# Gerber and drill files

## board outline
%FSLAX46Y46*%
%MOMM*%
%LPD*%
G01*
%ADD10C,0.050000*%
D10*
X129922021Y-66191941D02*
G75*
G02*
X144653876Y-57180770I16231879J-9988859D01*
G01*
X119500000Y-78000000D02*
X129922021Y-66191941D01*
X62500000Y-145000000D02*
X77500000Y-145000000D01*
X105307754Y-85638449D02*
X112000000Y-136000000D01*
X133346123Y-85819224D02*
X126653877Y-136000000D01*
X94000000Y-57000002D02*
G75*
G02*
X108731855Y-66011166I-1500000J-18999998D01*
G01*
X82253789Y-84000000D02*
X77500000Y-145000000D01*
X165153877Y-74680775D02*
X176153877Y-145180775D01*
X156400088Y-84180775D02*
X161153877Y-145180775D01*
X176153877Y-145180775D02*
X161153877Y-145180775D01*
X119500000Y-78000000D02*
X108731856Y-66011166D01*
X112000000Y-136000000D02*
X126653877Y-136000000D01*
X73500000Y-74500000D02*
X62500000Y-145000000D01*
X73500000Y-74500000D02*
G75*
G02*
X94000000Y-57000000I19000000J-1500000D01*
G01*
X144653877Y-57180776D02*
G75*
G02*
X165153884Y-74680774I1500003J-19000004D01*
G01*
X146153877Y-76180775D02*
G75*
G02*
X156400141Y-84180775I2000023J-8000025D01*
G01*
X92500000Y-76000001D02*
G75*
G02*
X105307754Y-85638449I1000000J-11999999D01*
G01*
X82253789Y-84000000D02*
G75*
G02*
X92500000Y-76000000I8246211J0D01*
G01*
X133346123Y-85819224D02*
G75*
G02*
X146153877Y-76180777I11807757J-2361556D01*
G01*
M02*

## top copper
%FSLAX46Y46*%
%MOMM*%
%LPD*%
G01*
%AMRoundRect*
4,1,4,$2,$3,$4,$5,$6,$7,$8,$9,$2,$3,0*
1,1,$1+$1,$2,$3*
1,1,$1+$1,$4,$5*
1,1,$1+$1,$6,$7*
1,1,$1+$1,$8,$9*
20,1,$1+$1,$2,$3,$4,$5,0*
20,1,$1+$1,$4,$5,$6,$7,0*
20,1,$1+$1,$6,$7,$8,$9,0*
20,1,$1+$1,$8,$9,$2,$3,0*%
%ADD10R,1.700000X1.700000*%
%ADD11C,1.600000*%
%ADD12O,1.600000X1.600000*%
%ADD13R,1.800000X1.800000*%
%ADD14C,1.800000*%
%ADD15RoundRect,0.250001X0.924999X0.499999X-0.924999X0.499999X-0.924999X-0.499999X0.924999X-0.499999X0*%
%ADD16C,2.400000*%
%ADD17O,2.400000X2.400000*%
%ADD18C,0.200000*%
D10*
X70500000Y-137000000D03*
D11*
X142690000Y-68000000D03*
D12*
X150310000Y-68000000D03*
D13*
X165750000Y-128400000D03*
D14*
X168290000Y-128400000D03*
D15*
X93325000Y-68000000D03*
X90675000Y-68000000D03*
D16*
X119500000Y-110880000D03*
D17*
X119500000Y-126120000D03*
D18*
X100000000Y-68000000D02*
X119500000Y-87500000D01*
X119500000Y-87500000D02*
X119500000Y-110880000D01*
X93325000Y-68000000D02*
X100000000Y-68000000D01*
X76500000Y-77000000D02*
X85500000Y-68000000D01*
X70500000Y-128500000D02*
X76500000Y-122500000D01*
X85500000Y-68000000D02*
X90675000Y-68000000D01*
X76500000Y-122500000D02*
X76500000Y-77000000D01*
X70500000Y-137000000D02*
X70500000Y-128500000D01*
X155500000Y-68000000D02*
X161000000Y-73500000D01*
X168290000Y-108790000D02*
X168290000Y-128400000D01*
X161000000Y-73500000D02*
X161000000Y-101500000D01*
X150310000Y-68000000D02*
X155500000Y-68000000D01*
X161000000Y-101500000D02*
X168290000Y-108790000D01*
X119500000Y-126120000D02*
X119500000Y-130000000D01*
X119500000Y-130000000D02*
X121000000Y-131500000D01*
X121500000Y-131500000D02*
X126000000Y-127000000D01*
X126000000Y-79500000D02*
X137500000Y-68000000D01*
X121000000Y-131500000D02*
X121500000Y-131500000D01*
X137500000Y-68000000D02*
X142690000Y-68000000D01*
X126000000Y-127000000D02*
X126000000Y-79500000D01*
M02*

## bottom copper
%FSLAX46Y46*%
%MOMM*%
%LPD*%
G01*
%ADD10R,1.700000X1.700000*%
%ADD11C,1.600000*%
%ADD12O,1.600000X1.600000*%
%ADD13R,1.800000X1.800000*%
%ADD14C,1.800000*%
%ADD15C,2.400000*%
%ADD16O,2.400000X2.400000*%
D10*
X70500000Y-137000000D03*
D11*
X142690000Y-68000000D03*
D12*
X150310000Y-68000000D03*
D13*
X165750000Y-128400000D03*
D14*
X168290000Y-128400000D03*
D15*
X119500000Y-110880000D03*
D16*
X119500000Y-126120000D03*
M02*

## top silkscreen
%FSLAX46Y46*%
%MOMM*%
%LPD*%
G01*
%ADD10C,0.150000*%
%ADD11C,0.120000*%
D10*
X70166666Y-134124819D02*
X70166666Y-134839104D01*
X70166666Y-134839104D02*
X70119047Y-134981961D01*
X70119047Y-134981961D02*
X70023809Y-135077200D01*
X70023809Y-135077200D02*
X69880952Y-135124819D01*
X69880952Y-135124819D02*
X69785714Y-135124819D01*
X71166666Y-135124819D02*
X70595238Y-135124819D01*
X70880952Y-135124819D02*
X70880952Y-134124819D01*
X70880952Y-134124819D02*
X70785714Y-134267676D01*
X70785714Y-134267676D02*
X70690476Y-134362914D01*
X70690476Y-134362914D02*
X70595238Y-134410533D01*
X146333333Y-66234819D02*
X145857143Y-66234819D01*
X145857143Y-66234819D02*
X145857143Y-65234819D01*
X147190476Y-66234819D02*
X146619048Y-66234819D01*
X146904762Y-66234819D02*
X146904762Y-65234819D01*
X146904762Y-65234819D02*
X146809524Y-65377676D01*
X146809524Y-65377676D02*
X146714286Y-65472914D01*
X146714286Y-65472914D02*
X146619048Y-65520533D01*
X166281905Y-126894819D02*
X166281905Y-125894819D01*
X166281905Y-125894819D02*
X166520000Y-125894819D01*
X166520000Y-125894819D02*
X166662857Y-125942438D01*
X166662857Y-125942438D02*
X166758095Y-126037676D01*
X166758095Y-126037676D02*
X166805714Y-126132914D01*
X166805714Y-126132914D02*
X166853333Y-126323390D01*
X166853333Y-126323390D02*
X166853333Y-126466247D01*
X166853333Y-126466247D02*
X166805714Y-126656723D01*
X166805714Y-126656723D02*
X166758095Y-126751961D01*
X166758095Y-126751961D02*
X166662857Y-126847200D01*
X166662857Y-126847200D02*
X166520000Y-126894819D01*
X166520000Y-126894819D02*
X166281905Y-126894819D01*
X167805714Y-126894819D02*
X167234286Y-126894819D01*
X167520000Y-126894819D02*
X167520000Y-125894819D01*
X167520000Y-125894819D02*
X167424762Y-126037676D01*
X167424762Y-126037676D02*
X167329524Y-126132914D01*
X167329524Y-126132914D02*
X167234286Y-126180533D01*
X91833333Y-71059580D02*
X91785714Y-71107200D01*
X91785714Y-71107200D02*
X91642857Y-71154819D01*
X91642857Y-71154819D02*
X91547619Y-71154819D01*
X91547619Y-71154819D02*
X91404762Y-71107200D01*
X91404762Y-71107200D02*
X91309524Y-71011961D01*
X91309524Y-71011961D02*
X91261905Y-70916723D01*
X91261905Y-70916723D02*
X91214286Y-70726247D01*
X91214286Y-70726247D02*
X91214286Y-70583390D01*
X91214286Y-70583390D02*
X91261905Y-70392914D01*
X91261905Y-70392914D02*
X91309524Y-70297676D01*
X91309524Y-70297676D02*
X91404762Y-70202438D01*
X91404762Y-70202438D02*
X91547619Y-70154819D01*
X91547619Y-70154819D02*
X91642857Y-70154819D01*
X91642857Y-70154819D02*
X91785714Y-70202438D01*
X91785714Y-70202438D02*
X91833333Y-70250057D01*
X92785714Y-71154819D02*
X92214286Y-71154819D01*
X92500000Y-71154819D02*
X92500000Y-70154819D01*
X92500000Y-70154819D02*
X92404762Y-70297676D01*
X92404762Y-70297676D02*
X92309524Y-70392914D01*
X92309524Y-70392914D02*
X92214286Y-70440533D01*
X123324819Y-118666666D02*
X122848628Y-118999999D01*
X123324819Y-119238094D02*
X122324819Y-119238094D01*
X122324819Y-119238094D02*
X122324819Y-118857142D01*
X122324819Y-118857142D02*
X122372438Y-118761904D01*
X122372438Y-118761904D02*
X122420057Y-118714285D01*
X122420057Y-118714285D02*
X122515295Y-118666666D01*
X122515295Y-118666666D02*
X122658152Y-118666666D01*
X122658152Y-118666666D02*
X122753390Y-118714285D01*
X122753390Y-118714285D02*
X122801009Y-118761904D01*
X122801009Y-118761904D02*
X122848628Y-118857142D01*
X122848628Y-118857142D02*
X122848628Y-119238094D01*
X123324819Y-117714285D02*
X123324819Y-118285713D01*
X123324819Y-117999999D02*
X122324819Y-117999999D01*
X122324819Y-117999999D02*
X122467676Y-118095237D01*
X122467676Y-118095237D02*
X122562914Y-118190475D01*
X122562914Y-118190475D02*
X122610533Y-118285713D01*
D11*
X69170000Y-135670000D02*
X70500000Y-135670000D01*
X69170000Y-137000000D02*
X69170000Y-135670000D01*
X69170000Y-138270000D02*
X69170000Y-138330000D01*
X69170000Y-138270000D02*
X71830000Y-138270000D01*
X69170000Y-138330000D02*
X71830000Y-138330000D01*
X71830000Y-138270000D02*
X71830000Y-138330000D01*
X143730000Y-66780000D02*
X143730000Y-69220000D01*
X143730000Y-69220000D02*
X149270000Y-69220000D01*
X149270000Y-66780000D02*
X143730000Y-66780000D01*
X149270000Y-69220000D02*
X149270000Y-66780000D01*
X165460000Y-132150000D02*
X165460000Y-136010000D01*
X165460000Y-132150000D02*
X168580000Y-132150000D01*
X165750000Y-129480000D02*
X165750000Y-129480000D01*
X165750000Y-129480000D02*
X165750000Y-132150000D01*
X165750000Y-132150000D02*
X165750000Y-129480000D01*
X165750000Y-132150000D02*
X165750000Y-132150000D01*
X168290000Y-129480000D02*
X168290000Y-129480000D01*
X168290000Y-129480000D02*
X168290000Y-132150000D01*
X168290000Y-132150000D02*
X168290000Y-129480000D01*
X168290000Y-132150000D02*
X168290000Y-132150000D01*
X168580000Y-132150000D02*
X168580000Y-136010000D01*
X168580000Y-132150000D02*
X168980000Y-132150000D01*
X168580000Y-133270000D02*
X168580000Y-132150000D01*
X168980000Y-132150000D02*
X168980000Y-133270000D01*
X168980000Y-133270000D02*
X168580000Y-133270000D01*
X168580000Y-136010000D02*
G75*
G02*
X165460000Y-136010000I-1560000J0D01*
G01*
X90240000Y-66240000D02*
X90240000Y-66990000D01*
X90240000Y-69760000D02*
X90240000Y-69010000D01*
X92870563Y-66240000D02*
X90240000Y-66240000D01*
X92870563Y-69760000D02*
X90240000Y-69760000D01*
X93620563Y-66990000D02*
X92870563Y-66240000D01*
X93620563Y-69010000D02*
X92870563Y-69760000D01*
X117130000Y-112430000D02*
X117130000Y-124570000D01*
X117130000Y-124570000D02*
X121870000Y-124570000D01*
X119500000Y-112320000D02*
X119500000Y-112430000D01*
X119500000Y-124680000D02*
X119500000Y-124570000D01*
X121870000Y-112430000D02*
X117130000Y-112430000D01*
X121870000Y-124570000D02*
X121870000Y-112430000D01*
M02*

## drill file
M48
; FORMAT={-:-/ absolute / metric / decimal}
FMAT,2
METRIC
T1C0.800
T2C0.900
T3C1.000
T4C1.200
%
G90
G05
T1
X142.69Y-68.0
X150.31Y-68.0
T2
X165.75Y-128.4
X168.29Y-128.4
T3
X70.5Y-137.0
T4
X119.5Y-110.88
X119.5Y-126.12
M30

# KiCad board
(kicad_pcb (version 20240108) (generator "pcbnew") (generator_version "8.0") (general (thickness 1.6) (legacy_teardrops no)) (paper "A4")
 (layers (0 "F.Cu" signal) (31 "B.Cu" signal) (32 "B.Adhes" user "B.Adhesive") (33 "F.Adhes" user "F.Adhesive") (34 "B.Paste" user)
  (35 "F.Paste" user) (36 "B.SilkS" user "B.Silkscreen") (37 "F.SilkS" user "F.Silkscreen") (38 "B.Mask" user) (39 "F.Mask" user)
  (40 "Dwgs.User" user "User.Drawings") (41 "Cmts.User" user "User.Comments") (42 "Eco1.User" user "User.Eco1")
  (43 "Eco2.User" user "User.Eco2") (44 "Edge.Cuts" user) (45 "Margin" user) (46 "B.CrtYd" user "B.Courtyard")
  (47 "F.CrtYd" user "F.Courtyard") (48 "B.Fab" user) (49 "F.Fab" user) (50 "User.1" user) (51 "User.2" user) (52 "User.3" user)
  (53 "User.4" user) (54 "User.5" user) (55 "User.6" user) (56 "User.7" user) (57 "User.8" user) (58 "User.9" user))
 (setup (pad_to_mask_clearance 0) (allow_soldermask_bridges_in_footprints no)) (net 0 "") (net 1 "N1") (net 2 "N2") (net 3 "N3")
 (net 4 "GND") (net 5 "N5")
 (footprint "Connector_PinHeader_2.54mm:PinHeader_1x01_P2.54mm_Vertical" (layer "F.Cu") (at 70.5 137)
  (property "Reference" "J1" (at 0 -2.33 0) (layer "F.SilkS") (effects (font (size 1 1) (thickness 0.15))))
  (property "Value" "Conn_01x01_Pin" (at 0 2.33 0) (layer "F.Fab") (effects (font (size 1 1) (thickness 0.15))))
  (fp_line (start -1.33 -1.33) (end 0 -1.33) (stroke (width 0.12) (type solid)) (layer "F.SilkS"))
  (fp_line (start -1.33 0) (end -1.33 -1.33) (stroke (width 0.12) (type solid)) (layer "F.SilkS"))
  (fp_line (start -1.33 1.27) (end -1.33 1.33) (stroke (width 0.12) (type solid)) (layer "F.SilkS"))
  (fp_line (start -1.33 1.27) (end 1.33 1.27) (stroke (width 0.12) (type solid)) (layer "F.SilkS"))
  (fp_line (start -1.33 1.33) (end 1.33 1.33) (stroke (width 0.12) (type solid)) (layer "F.SilkS"))
  (fp_line (start 1.33 1.27) (end 1.33 1.33) (stroke (width 0.12) (type solid)) (layer "F.SilkS"))
  (pad "1" thru_hole rect (at 0 0) (size 1.7 1.7) (drill 1) (layers "*.Cu" "*.Mask") (remove_unused_layers no) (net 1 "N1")))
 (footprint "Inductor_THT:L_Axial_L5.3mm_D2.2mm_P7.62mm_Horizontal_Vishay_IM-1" (layer "F.Cu") (at 142.69 68)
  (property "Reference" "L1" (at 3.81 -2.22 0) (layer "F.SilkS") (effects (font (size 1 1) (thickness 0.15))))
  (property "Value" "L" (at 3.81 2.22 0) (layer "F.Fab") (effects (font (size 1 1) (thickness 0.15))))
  (fp_line (start 1.04 -1.22) (end 1.04 1.22) (stroke (width 0.12) (type solid)) (layer "F.SilkS"))
  (fp_line (start 1.04 1.22) (end 6.58 1.22) (stroke (width 0.12) (type solid)) (layer "F.SilkS"))
  (fp_line (start 6.58 -1.22) (end 1.04 -1.22) (stroke (width 0.12) (type solid)) (layer "F.SilkS"))
  (fp_line (start 6.58 1.22) (end 6.58 -1.22) (stroke (width 0.12) (type solid)) (layer "F.SilkS"))
  (pad "1" thru_hole circle (at 0 0) (size 1.6 1.6) (drill 0.8) (layers "*.Cu" "*.Mask") (remove_unused_layers no) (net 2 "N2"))
  (pad "2" thru_hole oval (at 7.62 0) (size 1.6 1.6) (drill 0.8) (layers "*.Cu" "*.Mask") (remove_unused_layers no) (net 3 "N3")))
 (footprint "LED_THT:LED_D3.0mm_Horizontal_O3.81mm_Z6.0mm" (layer "F.Cu") (at 165.75 128.4)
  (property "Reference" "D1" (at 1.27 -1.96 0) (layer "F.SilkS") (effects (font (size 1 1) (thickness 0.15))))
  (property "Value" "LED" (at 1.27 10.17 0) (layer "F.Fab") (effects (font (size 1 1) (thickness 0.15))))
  (fp_line (start -0.29 3.75) (end -0.29 7.61) (stroke (width 0.12) (type solid)) (layer "F.SilkS"))
  (fp_line (start -0.29 3.75) (end 2.83 3.75) (stroke (width 0.12) (type solid)) (layer "F.SilkS"))
  (fp_line (start 0 1.08) (end 0 1.08) (stroke (width 0.12) (type solid)) (layer "F.SilkS"))
  (fp_line (start 0 1.08) (end 0 3.75) (stroke (width 0.12) (type solid)) (layer "F.SilkS"))
  (fp_line (start 0 3.75) (end 0 1.08) (stroke (width 0.12) (type solid)) (layer "F.SilkS"))
  (fp_line (start 0 3.75) (end 0 3.75) (stroke (width 0.12) (type solid)) (layer "F.SilkS"))
  (fp_line (start 2.54 1.08) (end 2.54 1.08) (stroke (width 0.12) (type solid)) (layer "F.SilkS"))
  (fp_line (start 2.54 1.08) (end 2.54 3.75) (stroke (width 0.12) (type solid)) (layer "F.SilkS"))
  (fp_line (start 2.54 3.75) (end 2.54 1.08) (stroke (width 0.12) (type solid)) (layer "F.SilkS"))
  (fp_line (start 2.54 3.75) (end 2.54 3.75) (stroke (width 0.12) (type solid)) (layer "F.SilkS"))
  (fp_line (start 2.83 3.75) (end 2.83 7.61) (stroke (width 0.12) (type solid)) (layer "F.SilkS"))
  (fp_line (start 2.83 3.75) (end 3.23 3.75) (stroke (width 0.12) (type solid)) (layer "F.SilkS"))
  (fp_line (start 2.83 4.87) (end 2.83 3.75) (stroke (width 0.12) (type solid)) (layer "F.SilkS"))
  (fp_line (start 3.23 3.75) (end 3.23 4.87) (stroke (width 0.12) (type solid)) (layer "F.SilkS"))
  (fp_line (start 3.23 4.87) (end 2.83 4.87) (stroke (width 0.12) (type solid)) (layer "F.SilkS"))
  (fp_arc (start 2.83 7.61) (mid 1.27 9.17) (end -0.29 7.61) (stroke (width 0.12) (type solid)) (layer "F.SilkS"))
  (pad "1" thru_hole rect (at 0 0) (size 1.8 1.8) (drill 0.9) (layers "*.Cu" "*.Mask") (remove_unused_layers no) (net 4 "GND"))
  (pad "2" thru_hole circle (at 2.54 0) (size 1.8 1.8) (drill 0.9) (layers "*.Cu" "*.Mask") (remove_unused_layers no) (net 3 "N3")))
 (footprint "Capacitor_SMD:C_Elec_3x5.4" (layer "F.Cu") (at 92 68 180)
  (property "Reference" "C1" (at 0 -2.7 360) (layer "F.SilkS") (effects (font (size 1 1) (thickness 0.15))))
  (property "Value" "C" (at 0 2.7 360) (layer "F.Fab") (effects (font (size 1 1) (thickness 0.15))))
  (fp_line (start 1.76 1.76) (end 1.76 1.01) (stroke (width 0.12) (type solid)) (layer "F.SilkS"))
  (fp_line (start 1.76 -1.76) (end 1.76 -1.01) (stroke (width 0.12) (type solid)) (layer "F.SilkS"))
  (fp_line (start -0.870563 1.76) (end 1.76 1.76) (stroke (width 0.12) (type solid)) (layer "F.SilkS"))
  (fp_line (start -0.870563 -1.76) (end 1.76 -1.76) (stroke (width 0.12) (type solid)) (layer "F.SilkS"))
  (fp_line (start -1.620563 1.01) (end -0.870563 1.76) (stroke (width 0.12) (type solid)) (layer "F.SilkS"))
  (fp_line (start -1.620563 -1.01) (end -0.870563 -1.76) (stroke (width 0.12) (type solid)) (layer "F.SilkS"))
  (pad "1" smd roundrect (at -1.325 0 180) (size 2.35 1.5) (layers "F.Cu" "F.Paste" "F.Mask") (roundrect_rratio 0.166667) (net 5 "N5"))
  (pad "2" smd roundrect (at 1.325 0 180) (size 2.35 1.5) (layers "F.Cu" "F.Paste" "F.Mask") (roundrect_rratio 0.166667) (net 1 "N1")))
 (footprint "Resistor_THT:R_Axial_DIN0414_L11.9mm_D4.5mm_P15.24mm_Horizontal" (layer "F.Cu") (at 119.5 110.88 -90)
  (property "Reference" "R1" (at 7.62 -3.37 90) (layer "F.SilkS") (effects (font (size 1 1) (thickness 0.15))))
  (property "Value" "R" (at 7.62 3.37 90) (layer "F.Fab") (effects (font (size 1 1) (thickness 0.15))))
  (fp_line (start 1.55 2.37) (end 13.69 2.37) (stroke (width 0.12) (type solid)) (layer "F.SilkS"))
  (fp_line (start 13.69 2.37) (end 13.69 -2.37) (stroke (width 0.12) (type solid)) (layer "F.SilkS"))
  (fp_line (start 1.44 0) (end 1.55 0) (stroke (width 0.12) (type solid)) (layer "F.SilkS"))
  (fp_line (start 13.8 0) (end 13.69 0) (stroke (width 0.12) (type solid)) (layer "F.SilkS"))
  (fp_line (start 1.55 -2.37) (end 1.55 2.37) (stroke (width 0.12) (type solid)) (layer "F.SilkS"))
  (fp_line (start 13.69 -2.37) (end 1.55 -2.37) (stroke (width 0.12) (type solid)) (layer "F.SilkS"))
  (pad "1" thru_hole circle (at 0 0 270) (size 2.4 2.4) (drill 1.2) (layers "*.Cu" "*.Mask") (remove_unused_layers no) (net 5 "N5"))
  (pad "2" thru_hole oval (at 15.24 0 270) (size 2.4 2.4) (drill 1.2) (layers "*.Cu" "*.Mask") (remove_unused_layers no) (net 2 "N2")))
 (gr_arc (start 129.922021 66.191941) (mid 136.20878 59.922086) (end 144.653877 57.180777) (stroke (width 0.05) (type default))
  (layer "Edge.Cuts"))
 (gr_line (start 119.5 78) (end 129.922021 66.191941) (stroke (width 0.05) (type default)) (layer "Edge.Cuts"))
 (gr_line (start 62.5 145) (end 77.5 145) (stroke (width 0.05) (type default)) (layer "Edge.Cuts"))
 (gr_line (start 105.307754 85.638449) (end 112 136) (stroke (width 0.05) (type default)) (layer "Edge.Cuts"))
 (gr_line (start 133.346123 85.819224) (end 126.653877 136) (stroke (width 0.05) (type default)) (layer "Edge.Cuts"))
 (gr_arc (start 94 57.000002) (mid 102.445097 59.741311) (end 108.731856 66.011166) (stroke (width 0.05) (type default)) (layer "Edge.Cuts"))
 (gr_line (start 82.253789 84) (end 77.5 145) (stroke (width 0.05) (type default)) (layer "Edge.Cuts"))
 (gr_line (start 165.153877 74.680775) (end 176.153877 145.180775) (stroke (width 0.05) (type default)) (layer "Edge.Cuts"))
 (gr_line (start 156.400088 84.180775) (end 161.153877 145.180775) (stroke (width 0.05) (type default)) (layer "Edge.Cuts"))
 (gr_line (start 176.153877 145.180775) (end 161.153877 145.180775) (stroke (width 0.05) (type default)) (layer "Edge.Cuts"))
 (gr_line (start 119.5 78) (end 108.731856 66.011166) (stroke (width 0.05) (type default)) (layer "Edge.Cuts"))
 (gr_line (start 112 136) (end 126.653877 136) (stroke (width 0.05) (type default)) (layer "Edge.Cuts"))
 (gr_line (start 73.5 74.5) (end 62.5 145) (stroke (width 0.05) (type default)) (layer "Edge.Cuts"))
 (gr_arc (start 73.5 74.5) (mid 80.125632 61.504312) (end 94 57.000001) (stroke (width 0.05) (type default)) (layer "Edge.Cuts"))
 (gr_arc (start 144.653877 57.180776) (mid 158.528245 61.685087) (end 165.153877 74.680775) (stroke (width 0.05) (type default))
  (layer "Edge.Cuts"))
 (gr_arc (start 146.153877 76.180775) (mid 153.228696 77.681067) (end 156.400088 84.180775) (stroke (width 0.05) (type default))
  (layer "Edge.Cuts"))
 (gr_arc (start 92.5 76.000001) (mid 100.740636 78.378505) (end 105.307754 85.638449) (stroke (width 0.05) (type default))
  (layer "Edge.Cuts"))
 (gr_arc (start 82.253789 84) (mid 85.425181 77.500292) (end 92.5 76) (stroke (width 0.05) (type default)) (layer "Edge.Cuts"))
 (gr_arc (start 133.346123 85.819224) (mid 137.913241 78.55928) (end 146.153877 76.180776) (stroke (width 0.05) (type default))
  (layer "Edge.Cuts"))
 (segment (start 100 68) (end 119.5 87.5) (width 0.2) (layer "F.Cu") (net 5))
 (segment (start 119.5 87.5) (end 119.5 110.88) (width 0.2) (layer "F.Cu") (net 5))
 (segment (start 93.325 68) (end 100 68) (width 0.2) (layer "F.Cu") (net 5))
 (segment (start 76.5 77) (end 85.5 68) (width 0.2) (layer "F.Cu") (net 1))
 (segment (start 70.5 128.5) (end 76.5 122.5) (width 0.2) (layer "F.Cu") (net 1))
 (segment (start 85.5 68) (end 90.675 68) (width 0.2) (layer "F.Cu") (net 1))
 (segment (start 76.5 122.5) (end 76.5 77) (width 0.2) (layer "F.Cu") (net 1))
 (segment (start 70.5 137) (end 70.5 128.5) (width 0.2) (layer "F.Cu") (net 1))
 (segment (start 155.5 68) (end 161 73.5) (width 0.2) (layer "F.Cu") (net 3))
 (segment (start 168.29 108.79) (end 168.29 128.4) (width 0.2) (layer "F.Cu") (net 3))
 (segment (start 161 73.5) (end 161 101.5) (width 0.2) (layer "F.Cu") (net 3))
 (segment (start 150.31 68) (end 155.5 68) (width 0.2) (layer "F.Cu") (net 3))
 (segment (start 161 101.5) (end 168.29 108.79) (width 0.2) (layer "F.Cu") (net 3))
 (segment (start 119.5 126.12) (end 119.5 130) (width 0.2) (layer "F.Cu") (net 2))
 (segment (start 119.5 130) (end 121 131.5) (width 0.2) (layer "F.Cu") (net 2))
 (segment (start 121.5 131.5) (end 126 127) (width 0.2) (layer "F.Cu") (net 2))
 (segment (start 126 79.5) (end 137.5 68) (width 0.2) (layer "F.Cu") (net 2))
 (segment (start 121 131.5) (end 121.5 131.5) (width 0.2) (layer "F.Cu") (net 2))
 (segment (start 137.5 68) (end 142.69 68) (width 0.2) (layer "F.Cu") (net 2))
 (segment (start 126 127) (end 126 79.5) (width 0.2) (layer "F.Cu") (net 2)))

